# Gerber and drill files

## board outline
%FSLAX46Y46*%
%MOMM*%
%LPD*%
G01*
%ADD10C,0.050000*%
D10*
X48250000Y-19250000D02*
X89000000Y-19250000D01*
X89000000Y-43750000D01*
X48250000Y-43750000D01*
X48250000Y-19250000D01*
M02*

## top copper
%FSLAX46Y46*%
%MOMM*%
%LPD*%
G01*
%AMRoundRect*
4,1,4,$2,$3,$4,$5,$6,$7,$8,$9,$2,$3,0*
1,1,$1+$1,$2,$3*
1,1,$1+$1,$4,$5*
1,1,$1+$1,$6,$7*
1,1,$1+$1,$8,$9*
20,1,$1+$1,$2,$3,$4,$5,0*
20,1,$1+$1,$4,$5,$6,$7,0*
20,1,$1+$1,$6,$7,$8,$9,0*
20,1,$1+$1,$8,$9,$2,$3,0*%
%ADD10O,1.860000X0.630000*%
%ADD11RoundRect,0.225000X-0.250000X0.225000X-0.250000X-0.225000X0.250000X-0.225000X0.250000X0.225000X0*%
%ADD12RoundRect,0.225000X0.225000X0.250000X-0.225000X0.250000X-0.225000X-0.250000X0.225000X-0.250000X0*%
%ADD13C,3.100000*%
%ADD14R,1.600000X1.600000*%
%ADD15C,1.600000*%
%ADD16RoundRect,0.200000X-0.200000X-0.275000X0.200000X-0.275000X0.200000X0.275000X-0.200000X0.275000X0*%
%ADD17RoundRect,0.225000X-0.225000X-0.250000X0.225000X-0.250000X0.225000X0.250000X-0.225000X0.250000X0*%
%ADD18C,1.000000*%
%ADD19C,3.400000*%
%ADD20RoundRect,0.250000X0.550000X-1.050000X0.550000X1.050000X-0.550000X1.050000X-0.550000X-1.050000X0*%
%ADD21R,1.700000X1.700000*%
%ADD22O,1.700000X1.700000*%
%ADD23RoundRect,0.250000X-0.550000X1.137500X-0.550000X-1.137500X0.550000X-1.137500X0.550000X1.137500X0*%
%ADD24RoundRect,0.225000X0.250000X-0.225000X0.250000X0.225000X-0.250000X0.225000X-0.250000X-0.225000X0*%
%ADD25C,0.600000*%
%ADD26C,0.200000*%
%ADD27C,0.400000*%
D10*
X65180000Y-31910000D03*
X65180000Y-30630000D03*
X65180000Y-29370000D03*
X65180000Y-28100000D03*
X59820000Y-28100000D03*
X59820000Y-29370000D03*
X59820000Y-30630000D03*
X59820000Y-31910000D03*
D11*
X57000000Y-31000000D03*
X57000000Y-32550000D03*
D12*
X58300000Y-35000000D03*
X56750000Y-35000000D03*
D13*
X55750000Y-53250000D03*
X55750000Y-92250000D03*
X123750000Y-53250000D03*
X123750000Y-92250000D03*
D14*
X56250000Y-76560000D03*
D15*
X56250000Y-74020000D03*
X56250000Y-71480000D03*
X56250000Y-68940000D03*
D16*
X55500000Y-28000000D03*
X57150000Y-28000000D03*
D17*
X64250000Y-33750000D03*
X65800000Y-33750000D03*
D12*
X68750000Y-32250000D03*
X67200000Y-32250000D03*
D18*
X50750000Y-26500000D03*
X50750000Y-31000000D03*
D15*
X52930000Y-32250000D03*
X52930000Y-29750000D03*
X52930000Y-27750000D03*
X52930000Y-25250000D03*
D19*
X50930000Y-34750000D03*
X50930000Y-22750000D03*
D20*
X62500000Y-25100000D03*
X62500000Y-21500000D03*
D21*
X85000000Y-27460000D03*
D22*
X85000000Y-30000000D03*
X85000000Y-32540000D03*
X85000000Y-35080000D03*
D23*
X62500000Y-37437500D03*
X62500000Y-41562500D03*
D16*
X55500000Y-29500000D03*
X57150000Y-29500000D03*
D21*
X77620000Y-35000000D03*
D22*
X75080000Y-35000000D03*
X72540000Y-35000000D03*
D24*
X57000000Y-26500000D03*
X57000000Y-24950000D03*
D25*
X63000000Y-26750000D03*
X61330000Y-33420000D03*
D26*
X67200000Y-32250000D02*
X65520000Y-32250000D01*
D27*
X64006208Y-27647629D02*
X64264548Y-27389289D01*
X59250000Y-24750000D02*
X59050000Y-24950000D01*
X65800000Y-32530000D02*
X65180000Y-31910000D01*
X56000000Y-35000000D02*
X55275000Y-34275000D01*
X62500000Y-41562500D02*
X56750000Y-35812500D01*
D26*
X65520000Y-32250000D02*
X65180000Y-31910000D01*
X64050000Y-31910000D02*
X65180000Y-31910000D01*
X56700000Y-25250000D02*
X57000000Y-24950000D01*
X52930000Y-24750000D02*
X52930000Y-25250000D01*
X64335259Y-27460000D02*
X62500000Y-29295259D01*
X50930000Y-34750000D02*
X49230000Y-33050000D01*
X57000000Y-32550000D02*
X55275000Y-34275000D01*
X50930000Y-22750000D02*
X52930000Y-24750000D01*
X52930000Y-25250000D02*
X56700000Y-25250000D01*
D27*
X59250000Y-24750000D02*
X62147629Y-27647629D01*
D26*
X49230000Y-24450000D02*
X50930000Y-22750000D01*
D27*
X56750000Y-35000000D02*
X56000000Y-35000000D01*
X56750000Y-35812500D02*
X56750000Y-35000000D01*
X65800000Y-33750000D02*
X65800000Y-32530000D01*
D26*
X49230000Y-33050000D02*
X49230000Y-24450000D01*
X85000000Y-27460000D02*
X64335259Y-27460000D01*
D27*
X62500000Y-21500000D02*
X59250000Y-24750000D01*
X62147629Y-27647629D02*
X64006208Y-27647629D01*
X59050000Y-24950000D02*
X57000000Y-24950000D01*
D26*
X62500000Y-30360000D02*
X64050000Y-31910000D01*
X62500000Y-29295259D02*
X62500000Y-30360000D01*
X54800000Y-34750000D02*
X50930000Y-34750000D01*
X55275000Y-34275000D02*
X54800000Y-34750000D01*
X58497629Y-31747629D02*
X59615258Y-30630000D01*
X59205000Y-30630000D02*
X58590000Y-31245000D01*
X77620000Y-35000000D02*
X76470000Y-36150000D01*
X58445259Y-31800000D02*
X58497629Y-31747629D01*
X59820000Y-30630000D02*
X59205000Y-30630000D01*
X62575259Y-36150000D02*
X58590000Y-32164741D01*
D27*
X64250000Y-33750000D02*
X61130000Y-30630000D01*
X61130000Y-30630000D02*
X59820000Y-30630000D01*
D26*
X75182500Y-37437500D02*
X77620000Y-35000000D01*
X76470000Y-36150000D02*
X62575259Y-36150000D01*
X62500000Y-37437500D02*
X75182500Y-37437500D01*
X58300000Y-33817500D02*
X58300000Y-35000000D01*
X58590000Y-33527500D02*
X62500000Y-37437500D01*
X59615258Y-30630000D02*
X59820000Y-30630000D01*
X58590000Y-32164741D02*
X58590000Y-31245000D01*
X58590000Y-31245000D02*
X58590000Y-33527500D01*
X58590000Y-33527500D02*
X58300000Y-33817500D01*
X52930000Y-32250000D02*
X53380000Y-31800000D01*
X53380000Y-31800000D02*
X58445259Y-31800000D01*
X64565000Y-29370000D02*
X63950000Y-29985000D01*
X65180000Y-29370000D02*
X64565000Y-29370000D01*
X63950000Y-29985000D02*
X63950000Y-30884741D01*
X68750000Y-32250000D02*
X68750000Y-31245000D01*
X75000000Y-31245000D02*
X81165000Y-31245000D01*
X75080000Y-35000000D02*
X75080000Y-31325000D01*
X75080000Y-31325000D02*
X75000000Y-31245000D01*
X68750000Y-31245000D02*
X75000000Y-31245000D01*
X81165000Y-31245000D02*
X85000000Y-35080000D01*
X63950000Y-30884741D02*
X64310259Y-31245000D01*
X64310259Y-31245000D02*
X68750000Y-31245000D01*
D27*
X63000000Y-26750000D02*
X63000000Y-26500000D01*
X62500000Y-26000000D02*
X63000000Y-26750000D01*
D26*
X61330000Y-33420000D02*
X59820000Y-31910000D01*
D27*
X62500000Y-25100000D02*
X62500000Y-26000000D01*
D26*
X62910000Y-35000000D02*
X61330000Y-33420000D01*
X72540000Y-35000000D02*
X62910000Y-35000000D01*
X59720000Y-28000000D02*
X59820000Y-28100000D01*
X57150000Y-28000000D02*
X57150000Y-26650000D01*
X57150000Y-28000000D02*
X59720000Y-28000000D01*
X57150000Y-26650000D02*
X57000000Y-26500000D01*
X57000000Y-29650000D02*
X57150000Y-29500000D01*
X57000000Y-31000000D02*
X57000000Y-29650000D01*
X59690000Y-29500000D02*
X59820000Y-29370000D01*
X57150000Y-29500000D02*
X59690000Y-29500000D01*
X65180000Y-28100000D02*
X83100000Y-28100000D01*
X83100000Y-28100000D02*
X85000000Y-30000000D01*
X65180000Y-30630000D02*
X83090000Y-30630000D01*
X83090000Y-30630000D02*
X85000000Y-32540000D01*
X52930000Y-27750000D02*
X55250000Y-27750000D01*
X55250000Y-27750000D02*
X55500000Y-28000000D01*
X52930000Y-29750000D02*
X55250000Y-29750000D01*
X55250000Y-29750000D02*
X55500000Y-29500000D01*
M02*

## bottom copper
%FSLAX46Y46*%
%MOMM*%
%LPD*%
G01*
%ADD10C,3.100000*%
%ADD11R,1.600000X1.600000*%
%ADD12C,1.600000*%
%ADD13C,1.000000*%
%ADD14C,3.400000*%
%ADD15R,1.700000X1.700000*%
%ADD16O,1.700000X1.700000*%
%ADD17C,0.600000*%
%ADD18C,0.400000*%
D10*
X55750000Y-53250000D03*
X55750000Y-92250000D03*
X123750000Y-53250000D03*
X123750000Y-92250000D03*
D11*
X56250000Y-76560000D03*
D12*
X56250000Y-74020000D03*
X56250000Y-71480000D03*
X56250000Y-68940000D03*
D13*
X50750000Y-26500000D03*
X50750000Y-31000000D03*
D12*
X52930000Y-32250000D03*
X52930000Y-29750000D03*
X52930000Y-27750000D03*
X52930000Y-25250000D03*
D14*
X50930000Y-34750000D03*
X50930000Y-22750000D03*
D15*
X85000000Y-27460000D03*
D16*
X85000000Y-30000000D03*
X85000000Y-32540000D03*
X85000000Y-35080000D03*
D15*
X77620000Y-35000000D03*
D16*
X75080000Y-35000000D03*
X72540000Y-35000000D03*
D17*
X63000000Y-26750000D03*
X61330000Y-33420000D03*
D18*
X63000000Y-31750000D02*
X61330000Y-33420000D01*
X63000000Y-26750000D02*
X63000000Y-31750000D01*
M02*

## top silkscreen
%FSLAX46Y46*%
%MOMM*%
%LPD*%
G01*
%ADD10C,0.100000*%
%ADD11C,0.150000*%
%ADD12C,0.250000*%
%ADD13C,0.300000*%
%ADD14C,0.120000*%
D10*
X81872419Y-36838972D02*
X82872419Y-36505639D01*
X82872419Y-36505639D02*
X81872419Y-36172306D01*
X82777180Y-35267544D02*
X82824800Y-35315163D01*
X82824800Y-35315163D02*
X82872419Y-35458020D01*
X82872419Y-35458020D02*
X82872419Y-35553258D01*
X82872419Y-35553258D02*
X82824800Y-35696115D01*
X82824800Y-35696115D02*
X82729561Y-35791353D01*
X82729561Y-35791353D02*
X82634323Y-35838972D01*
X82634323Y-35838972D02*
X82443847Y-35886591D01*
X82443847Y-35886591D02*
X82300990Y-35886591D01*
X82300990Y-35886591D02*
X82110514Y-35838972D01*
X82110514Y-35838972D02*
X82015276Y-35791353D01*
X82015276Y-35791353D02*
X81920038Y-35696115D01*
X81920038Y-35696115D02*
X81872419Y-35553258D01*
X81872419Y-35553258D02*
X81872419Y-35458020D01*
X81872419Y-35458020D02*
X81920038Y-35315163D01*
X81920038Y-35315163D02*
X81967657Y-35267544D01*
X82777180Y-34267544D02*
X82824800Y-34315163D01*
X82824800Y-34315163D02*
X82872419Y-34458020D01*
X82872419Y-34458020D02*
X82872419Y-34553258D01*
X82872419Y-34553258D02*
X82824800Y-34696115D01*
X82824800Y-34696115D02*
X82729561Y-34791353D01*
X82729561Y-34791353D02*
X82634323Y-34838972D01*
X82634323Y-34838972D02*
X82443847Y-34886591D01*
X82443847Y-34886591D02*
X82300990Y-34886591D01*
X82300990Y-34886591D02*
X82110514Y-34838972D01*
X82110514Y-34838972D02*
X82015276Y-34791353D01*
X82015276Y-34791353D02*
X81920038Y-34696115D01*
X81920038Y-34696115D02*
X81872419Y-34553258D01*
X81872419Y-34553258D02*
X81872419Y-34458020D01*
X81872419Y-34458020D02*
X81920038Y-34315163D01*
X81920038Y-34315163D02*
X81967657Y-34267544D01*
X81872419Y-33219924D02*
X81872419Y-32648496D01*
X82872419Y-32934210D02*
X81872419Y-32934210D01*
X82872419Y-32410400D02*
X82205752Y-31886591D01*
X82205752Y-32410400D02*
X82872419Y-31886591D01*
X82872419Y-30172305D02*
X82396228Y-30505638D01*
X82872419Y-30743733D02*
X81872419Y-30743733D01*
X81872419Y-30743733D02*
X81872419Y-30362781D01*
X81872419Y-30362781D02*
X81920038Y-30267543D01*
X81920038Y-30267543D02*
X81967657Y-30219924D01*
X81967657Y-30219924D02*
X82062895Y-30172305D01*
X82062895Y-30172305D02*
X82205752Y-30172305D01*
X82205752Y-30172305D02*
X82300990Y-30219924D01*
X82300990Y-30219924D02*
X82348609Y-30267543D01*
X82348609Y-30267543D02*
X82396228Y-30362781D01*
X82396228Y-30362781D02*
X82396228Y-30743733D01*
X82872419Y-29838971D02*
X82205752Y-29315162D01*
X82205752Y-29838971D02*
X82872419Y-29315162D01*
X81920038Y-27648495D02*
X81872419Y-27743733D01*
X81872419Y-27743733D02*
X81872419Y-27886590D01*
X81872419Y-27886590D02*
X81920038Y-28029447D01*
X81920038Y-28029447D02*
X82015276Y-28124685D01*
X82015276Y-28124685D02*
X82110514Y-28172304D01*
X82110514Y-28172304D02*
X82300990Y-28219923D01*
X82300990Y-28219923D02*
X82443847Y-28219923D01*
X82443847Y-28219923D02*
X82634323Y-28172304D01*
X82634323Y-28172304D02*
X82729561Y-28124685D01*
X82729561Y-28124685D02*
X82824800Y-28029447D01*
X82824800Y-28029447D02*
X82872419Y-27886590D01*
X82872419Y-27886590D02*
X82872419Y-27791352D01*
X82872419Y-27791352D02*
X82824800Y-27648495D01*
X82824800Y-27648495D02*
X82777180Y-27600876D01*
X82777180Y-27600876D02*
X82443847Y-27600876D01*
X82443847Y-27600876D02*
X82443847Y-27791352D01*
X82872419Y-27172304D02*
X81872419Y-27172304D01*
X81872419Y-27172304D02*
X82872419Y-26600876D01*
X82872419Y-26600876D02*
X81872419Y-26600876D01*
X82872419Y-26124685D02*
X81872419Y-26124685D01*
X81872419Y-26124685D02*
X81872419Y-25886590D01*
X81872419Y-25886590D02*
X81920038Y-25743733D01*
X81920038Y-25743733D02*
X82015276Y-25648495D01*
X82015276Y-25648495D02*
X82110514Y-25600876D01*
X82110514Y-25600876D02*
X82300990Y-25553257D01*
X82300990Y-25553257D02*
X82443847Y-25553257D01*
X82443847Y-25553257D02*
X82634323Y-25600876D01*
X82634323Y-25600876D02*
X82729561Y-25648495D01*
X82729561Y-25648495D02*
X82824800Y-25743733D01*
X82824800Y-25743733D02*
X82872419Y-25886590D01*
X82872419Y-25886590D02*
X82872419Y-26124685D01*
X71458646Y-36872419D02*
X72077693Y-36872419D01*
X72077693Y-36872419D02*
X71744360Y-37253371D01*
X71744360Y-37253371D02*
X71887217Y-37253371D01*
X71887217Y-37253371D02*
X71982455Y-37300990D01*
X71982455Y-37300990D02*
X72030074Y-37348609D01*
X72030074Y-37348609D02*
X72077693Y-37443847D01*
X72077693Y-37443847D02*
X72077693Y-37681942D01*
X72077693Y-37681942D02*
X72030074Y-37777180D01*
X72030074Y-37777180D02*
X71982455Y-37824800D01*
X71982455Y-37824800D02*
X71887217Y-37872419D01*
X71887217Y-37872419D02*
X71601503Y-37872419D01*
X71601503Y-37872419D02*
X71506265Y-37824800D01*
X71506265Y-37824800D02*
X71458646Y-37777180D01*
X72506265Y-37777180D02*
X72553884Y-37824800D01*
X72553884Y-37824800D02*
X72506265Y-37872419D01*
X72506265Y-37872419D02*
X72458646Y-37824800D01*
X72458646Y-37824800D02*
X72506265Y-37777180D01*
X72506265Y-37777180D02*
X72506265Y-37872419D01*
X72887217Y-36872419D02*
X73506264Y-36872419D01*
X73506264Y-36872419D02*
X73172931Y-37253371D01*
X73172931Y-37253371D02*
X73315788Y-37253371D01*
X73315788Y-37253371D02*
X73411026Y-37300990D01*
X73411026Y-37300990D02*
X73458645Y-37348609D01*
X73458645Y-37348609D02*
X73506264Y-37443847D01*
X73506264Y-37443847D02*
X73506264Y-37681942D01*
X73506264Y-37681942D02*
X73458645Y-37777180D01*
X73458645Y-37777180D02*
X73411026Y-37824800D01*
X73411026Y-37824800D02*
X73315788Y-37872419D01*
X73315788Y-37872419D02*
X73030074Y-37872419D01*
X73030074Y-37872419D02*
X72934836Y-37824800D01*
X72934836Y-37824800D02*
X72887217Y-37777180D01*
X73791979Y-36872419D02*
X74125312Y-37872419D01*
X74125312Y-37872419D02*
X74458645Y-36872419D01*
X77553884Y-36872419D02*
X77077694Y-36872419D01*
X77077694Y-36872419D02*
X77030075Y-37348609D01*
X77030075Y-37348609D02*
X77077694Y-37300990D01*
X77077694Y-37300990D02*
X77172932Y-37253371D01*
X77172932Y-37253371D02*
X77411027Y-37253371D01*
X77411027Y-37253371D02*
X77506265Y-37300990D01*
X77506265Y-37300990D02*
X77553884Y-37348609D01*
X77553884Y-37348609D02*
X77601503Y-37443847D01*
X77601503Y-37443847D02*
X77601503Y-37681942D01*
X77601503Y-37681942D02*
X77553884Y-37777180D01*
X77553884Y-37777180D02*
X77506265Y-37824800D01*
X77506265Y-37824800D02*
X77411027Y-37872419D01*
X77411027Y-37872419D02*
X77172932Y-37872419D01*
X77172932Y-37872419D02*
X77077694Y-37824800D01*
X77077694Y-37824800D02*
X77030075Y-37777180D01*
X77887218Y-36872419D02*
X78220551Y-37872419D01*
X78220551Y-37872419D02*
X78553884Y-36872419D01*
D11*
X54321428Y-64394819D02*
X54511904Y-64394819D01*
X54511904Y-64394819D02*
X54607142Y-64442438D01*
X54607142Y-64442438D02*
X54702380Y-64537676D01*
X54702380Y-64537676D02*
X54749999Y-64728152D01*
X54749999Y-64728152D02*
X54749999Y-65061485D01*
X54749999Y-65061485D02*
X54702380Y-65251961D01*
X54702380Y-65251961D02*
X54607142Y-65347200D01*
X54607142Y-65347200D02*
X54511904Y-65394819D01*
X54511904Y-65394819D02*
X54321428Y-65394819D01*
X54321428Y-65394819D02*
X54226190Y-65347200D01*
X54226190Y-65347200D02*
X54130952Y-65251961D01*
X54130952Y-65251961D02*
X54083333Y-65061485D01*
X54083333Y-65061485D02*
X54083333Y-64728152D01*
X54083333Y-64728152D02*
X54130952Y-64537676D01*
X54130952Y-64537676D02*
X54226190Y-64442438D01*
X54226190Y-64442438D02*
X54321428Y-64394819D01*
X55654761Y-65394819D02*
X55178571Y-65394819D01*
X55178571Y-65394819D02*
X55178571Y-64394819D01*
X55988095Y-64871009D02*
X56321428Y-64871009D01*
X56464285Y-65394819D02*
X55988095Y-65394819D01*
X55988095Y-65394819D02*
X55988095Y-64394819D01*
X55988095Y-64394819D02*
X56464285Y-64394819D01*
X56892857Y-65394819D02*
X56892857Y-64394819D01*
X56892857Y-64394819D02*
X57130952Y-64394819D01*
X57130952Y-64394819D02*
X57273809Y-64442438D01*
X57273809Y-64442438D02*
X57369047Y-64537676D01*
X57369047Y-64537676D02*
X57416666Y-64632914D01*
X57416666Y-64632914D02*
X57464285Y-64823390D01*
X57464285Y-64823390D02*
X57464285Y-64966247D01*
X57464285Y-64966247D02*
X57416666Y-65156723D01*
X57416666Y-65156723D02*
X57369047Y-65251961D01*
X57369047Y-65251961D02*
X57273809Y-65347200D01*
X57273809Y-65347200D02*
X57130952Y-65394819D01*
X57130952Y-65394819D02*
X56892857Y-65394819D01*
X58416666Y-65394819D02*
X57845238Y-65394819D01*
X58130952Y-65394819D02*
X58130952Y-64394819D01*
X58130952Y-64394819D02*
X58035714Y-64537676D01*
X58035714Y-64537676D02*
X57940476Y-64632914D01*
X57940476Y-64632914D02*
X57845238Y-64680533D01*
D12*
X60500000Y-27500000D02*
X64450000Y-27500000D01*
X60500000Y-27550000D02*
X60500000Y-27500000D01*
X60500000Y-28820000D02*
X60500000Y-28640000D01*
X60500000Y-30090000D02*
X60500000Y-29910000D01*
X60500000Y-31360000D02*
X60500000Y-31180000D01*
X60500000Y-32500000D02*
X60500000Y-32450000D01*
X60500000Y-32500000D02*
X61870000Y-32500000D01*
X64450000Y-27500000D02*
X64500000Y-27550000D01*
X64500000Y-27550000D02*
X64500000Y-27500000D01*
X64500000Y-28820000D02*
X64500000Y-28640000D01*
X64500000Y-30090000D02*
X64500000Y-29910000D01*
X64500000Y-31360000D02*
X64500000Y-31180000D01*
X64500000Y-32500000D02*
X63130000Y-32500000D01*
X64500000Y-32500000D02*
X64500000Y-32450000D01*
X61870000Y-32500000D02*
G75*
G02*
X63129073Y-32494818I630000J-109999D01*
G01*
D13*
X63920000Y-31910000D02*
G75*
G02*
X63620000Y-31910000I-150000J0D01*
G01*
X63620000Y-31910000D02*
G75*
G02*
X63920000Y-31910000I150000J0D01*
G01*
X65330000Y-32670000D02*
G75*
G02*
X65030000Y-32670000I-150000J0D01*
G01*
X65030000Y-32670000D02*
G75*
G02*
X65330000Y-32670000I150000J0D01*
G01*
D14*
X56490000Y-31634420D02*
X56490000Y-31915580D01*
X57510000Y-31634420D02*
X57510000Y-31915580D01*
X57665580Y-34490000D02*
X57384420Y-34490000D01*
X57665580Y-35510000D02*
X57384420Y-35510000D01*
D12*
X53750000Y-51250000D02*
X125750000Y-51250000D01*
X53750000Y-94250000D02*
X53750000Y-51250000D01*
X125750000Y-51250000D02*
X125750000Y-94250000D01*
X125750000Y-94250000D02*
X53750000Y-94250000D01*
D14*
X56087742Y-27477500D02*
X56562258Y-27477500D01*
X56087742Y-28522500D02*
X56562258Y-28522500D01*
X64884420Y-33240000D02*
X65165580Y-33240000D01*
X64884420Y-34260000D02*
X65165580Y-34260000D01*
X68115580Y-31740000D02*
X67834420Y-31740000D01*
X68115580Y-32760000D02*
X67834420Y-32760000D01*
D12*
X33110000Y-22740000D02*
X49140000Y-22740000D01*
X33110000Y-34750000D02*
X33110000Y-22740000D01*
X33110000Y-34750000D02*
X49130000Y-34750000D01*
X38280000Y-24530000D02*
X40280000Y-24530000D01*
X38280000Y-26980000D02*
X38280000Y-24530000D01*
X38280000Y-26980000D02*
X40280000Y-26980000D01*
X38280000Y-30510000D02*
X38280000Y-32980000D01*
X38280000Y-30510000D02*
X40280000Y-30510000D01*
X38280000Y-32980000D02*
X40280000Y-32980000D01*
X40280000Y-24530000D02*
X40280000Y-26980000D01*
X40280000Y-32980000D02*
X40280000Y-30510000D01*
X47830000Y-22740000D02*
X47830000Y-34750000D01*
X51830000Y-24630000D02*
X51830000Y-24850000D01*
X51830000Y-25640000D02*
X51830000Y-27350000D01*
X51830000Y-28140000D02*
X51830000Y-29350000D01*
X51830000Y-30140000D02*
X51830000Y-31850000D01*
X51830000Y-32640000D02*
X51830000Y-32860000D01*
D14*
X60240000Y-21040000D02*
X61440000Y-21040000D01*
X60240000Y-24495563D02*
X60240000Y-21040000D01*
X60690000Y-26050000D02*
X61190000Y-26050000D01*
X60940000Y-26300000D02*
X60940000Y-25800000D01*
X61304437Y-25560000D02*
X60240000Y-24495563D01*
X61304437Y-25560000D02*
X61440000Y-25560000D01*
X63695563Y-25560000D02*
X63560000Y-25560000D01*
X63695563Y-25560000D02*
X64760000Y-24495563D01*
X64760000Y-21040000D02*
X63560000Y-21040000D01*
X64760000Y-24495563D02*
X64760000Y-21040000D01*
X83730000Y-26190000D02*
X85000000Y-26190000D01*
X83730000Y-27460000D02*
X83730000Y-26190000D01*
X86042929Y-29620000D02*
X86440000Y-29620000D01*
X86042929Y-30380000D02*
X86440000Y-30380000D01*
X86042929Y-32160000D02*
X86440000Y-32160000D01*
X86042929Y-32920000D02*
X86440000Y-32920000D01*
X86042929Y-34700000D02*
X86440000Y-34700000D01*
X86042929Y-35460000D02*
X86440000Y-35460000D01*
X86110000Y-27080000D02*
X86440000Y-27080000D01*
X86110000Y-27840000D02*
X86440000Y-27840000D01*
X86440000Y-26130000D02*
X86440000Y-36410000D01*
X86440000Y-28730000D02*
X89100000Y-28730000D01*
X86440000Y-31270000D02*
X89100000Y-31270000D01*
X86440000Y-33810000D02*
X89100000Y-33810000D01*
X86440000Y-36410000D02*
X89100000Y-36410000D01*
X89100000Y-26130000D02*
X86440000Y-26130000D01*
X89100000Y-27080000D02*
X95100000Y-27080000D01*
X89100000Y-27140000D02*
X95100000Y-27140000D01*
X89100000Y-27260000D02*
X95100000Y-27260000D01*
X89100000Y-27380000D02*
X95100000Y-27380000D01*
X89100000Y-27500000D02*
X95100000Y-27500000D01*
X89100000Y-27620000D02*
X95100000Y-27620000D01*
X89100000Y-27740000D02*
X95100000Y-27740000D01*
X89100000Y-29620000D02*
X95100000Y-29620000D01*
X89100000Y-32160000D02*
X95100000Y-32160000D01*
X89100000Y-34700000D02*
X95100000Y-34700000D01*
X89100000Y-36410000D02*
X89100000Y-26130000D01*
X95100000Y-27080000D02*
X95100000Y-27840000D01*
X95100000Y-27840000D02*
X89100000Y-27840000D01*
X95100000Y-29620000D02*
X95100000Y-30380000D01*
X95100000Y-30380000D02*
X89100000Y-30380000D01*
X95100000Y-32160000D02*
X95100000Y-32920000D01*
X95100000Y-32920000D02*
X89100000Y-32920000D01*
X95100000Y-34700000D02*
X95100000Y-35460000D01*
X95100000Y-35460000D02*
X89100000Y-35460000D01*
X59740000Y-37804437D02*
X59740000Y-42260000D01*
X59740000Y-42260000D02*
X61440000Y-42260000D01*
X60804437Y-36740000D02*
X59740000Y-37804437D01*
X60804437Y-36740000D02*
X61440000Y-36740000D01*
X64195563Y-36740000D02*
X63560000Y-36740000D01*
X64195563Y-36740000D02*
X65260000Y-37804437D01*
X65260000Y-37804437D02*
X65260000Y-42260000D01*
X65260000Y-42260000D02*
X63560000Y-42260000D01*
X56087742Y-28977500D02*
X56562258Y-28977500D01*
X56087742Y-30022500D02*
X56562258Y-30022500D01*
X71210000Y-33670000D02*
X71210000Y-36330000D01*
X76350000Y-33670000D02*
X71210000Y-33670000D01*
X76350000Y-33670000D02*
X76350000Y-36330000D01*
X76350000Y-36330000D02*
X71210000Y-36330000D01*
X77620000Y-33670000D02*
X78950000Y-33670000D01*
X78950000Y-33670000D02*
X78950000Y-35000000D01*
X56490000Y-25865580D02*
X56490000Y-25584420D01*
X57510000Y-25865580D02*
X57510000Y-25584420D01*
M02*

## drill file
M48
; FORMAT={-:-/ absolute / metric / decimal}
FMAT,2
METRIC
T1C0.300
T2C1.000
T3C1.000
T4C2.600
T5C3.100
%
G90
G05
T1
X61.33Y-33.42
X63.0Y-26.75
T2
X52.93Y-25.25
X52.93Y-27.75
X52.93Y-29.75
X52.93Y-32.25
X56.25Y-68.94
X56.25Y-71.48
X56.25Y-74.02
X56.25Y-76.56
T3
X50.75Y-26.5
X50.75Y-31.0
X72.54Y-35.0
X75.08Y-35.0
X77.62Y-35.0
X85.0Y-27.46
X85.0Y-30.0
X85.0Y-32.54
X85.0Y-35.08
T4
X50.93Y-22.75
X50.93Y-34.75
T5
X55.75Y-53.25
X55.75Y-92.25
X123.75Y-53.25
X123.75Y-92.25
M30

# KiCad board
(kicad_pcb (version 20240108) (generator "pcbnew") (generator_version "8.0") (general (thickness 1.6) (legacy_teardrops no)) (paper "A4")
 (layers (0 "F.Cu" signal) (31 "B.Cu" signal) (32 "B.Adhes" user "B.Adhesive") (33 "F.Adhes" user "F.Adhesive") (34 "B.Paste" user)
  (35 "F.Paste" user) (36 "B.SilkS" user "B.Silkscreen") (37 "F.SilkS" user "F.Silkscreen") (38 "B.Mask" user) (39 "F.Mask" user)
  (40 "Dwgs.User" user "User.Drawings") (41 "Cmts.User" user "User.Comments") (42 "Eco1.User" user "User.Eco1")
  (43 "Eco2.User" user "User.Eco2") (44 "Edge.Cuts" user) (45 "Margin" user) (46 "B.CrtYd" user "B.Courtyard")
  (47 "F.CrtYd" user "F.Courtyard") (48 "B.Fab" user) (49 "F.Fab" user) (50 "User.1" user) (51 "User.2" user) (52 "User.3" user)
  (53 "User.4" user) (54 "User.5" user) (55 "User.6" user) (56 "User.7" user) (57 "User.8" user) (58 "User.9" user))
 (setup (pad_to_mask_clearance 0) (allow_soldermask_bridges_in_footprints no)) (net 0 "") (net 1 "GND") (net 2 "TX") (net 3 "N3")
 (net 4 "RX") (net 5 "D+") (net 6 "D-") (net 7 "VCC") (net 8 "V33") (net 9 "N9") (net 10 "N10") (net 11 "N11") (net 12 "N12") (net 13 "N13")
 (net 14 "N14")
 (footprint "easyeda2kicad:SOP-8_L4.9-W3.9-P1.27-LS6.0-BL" (layer "F.Cu") (at 62.5 30 90)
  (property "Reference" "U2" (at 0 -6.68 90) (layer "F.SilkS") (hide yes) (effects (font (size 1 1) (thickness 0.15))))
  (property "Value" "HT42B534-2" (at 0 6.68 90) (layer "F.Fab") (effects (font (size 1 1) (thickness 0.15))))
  (fp_line (start 2.5 -2) (end 2.5 1.95) (stroke (width 0.25) (type solid)) (layer "F.SilkS"))
  (fp_line (start 2.45 -2) (end 2.5 -2) (stroke (width 0.25) (type solid)) (layer "F.SilkS"))
  (fp_line (start 1.18 -2) (end 1.36 -2) (stroke (width 0.25) (type solid)) (layer "F.SilkS"))
  (fp_line (start -0.09 -2) (end 0.09 -2) (stroke (width 0.25) (type solid)) (layer "F.SilkS"))
  (fp_line (start -1.36 -2) (end -1.18 -2) (stroke (width 0.25) (type solid)) (layer "F.SilkS"))
  (fp_line (start -2.5 -2) (end -2.45 -2) (stroke (width 0.25) (type solid)) (layer "F.SilkS"))
  (fp_line (start -2.5 -2) (end -2.5 -0.63) (stroke (width 0.25) (type solid)) (layer "F.SilkS"))
  (fp_line (start 2.5 1.95) (end 2.45 2) (stroke (width 0.25) (type solid)) (layer "F.SilkS"))
  (fp_line (start 2.45 2) (end 2.5 2) (stroke (width 0.25) (type solid)) (layer "F.SilkS"))
  (fp_line (start 1.18 2) (end 1.36 2) (stroke (width 0.25) (type solid)) (layer "F.SilkS"))
  (fp_line (start -0.09 2) (end 0.09 2) (stroke (width 0.25) (type solid)) (layer "F.SilkS"))
  (fp_line (start -1.36 2) (end -1.18 2) (stroke (width 0.25) (type solid)) (layer "F.SilkS"))
  (fp_line (start -2.5 2) (end -2.5 0.63) (stroke (width 0.25) (type solid)) (layer "F.SilkS"))
  (fp_line (start -2.5 2) (end -2.45 2) (stroke (width 0.25) (type solid)) (layer "F.SilkS"))
  (fp_arc (start -2.5 -0.63) (mid -1.970474 -0.002632) (end -2.494818 0.629073) (stroke (width 0.25) (type solid)) (layer "F.SilkS"))
  (fp_circle (center -1.91 1.27) (end -1.76 1.27) (stroke (width 0.3) (type solid)) (fill none) (layer "F.SilkS"))
  (fp_circle (center -2.67 2.68) (end -2.52 2.68) (stroke (width 0.3) (type solid)) (fill none) (layer "F.SilkS"))
  (pad "1" smd oval (at -1.91 2.68 90) (size 0.63 1.86) (layers "F.Cu" "F.Paste" "F.Mask") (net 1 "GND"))
  (pad "2" smd oval (at -0.63 2.68 90) (size 0.63 1.86) (layers "F.Cu" "F.Paste" "F.Mask") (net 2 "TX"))
  (pad "3" smd oval (at 0.63 2.68 90) (size 0.63 1.86) (layers "F.Cu" "F.Paste" "F.Mask") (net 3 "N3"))
  (pad "4" smd oval (at 1.9 2.68 90) (size 0.63 1.86) (layers "F.Cu" "F.Paste" "F.Mask") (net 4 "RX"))
  (pad "5" smd oval (at 1.9 -2.68 90) (size 0.63 1.86) (layers "F.Cu" "F.Paste" "F.Mask") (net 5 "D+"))
  (pad "6" smd oval (at 0.63 -2.68 90) (size 0.63 1.86) (layers "F.Cu" "F.Paste" "F.Mask") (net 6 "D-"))
  (pad "7" smd oval (at -0.63 -2.68 90) (size 0.63 1.86) (layers "F.Cu" "F.Paste" "F.Mask") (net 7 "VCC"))
  (pad "8" smd oval (at -1.91 -2.68 90) (size 0.63 1.86) (layers "F.Cu" "F.Paste" "F.Mask") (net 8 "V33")))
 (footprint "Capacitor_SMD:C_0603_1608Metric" (layer "F.Cu") (at 57 31.775 -90)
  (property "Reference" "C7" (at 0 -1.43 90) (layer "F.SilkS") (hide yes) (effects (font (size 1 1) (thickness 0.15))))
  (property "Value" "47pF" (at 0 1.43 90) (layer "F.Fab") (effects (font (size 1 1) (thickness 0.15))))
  (fp_line (start -0.14058 0.51) (end 0.14058 0.51) (stroke (width 0.12) (type solid)) (layer "F.SilkS"))
  (fp_line (start -0.14058 -0.51) (end 0.14058 -0.51) (stroke (width 0.12) (type solid)) (layer "F.SilkS"))
  (pad "1" smd roundrect (at -0.775 0 270) (size 0.9 0.95) (layers "F.Cu" "F.Paste" "F.Mask") (roundrect_rratio 0.25) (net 6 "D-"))
  (pad "2" smd roundrect (at 0.775 0 270) (size 0.9 0.95) (layers "F.Cu" "F.Paste" "F.Mask") (roundrect_rratio 0.25) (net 1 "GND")))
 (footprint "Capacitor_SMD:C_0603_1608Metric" (layer "F.Cu") (at 57.525 35 180)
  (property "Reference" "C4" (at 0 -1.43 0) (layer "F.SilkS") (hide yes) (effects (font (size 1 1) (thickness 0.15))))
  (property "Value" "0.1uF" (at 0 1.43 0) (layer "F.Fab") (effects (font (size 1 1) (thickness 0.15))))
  (fp_line (start -0.14058 0.51) (end 0.14058 0.51) (stroke (width 0.12) (type solid)) (layer "F.SilkS"))
  (fp_line (start -0.14058 -0.51) (end 0.14058 -0.51) (stroke (width 0.12) (type solid)) (layer "F.SilkS"))
  (pad "1" smd roundrect (at -0.775 0 180) (size 0.9 0.95) (layers "F.Cu" "F.Paste" "F.Mask") (roundrect_rratio 0.25) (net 7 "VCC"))
  (pad "2" smd roundrect (at 0.775 0 180) (size 0.9 0.95) (layers "F.Cu" "F.Paste" "F.Mask") (roundrect_rratio 0.25) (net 1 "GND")))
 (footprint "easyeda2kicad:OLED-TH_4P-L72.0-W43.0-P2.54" (layer "F.Cu") (at 56.25 72.75)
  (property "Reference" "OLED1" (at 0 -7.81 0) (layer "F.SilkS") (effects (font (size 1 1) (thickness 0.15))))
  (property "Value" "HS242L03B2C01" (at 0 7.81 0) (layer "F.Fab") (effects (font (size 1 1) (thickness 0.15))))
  (fp_line (start -2.5 -21.5) (end 69.5 -21.5) (stroke (width 0.25) (type solid)) (layer "F.SilkS"))
  (fp_line (start -2.5 21.5) (end -2.5 -21.5) (stroke (width 0.25) (type solid)) (layer "F.SilkS"))
  (fp_line (start 69.5 -21.5) (end 69.5 21.5) (stroke (width 0.25) (type solid)) (layer "F.SilkS"))
  (fp_line (start 69.5 21.5) (end -2.5 21.5) (stroke (width 0.25) (type solid)) (layer "F.SilkS"))
  (pad "" thru_hole circle (at -0.5 -19.5) (size 3.1 3.1) (drill 3.1) (layers "*.Cu" "*.Mask") (remove_unused_layers no))
  (pad "" thru_hole circle (at -0.5 19.5) (size 3.1 3.1) (drill 3.1) (layers "*.Cu" "*.Mask") (remove_unused_layers no))
  (pad "" thru_hole circle (at 67.5 -19.5) (size 3.1 3.1) (drill 3.1) (layers "*.Cu" "*.Mask") (remove_unused_layers no))
  (pad "" thru_hole circle (at 67.5 19.5) (size 3.1 3.1) (drill 3.1) (layers "*.Cu" "*.Mask") (remove_unused_layers no))
  (pad "1" thru_hole rect (at 0 3.81) (size 1.6 1.6) (drill 0.999998) (layers "*.Cu" "*.Mask") (remove_unused_layers no) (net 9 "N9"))
  (pad "2" thru_hole circle (at 0 1.27) (size 1.6 1.6) (drill 0.999998) (layers "*.Cu" "*.Mask") (remove_unused_layers no) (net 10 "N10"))
  (pad "3" thru_hole circle (at 0 -1.27) (size 1.6 1.6) (drill 0.999998) (layers "*.Cu" "*.Mask") (remove_unused_layers no) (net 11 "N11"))
  (pad "4" thru_hole circle (at 0 -3.81) (size 1.6 1.6) (drill 0.999998) (layers "*.Cu" "*.Mask") (remove_unused_layers no) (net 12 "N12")))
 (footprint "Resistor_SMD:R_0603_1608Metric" (layer "F.Cu") (at 56.325 28)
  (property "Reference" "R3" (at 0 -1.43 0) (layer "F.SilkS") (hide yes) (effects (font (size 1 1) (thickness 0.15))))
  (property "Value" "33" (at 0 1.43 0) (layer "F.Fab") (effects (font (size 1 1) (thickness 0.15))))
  (fp_line (start -0.237258 -0.5225) (end 0.237258 -0.5225) (stroke (width 0.12) (type solid)) (layer "F.SilkS"))
  (fp_line (start -0.237258 0.5225) (end 0.237258 0.5225) (stroke (width 0.12) (type solid)) (layer "F.SilkS"))
  (pad "1" smd roundrect (at -0.825 0) (size 0.8 0.95) (layers "F.Cu" "F.Paste" "F.Mask") (roundrect_rratio 0.25) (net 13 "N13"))
  (pad "2" smd roundrect (at 0.825 0) (size 0.8 0.95) (layers "F.Cu" "F.Paste" "F.Mask") (roundrect_rratio 0.25) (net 5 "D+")))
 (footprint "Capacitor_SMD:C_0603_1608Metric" (layer "F.Cu") (at 65.025 33.75)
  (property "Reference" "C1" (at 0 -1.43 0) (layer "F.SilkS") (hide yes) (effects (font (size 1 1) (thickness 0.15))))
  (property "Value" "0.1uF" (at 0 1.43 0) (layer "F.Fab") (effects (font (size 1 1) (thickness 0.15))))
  (fp_line (start -0.14058 -0.51) (end 0.14058 -0.51) (stroke (width 0.12) (type solid)) (layer "F.SilkS"))
  (fp_line (start -0.14058 0.51) (end 0.14058 0.51) (stroke (width 0.12) (type solid)) (layer "F.SilkS"))
  (pad "1" smd roundrect (at -0.775 0) (size 0.9 0.95) (layers "F.Cu" "F.Paste" "F.Mask") (roundrect_rratio 0.25) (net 7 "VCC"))
  (pad "2" smd roundrect (at 0.775 0) (size 0.9 0.95) (layers "F.Cu" "F.Paste" "F.Mask") (roundrect_rratio 0.25) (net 1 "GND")))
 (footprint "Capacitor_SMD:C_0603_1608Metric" (layer "F.Cu") (at 67.975 32.25 180)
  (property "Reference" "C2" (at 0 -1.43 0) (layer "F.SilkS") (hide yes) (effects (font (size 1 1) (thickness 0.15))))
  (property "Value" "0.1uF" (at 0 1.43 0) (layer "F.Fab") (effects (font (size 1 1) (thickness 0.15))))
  (fp_line (start -0.14058 0.51) (end 0.14058 0.51) (stroke (width 0.12) (type solid)) (layer "F.SilkS"))
  (fp_line (start -0.14058 -0.51) (end 0.14058 -0.51) (stroke (width 0.12) (type solid)) (layer "F.SilkS"))
  (pad "1" smd roundrect (at -0.775 0 180) (size 0.9 0.95) (layers "F.Cu" "F.Paste" "F.Mask") (roundrect_rratio 0.25) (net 3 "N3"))
  (pad "2" smd roundrect (at 0.775 0 180) (size 0.9 0.95) (layers "F.Cu" "F.Paste" "F.Mask") (roundrect_rratio 0.25) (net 1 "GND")))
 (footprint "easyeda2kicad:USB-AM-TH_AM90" (layer "F.Cu") (at 51.93 28.75 -90)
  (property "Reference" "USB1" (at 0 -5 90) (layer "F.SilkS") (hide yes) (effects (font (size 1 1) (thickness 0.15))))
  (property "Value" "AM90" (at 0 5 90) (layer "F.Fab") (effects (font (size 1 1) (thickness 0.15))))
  (fp_line (start -6.01 18.82) (end -6.01 2.79) (stroke (width 0.25) (type solid)) (layer "F.SilkS"))
  (fp_line (start 6 18.82) (end -6.01 18.82) (stroke (width 0.25) (type solid)) (layer "F.SilkS"))
  (fp_line (start 6 18.82) (end 6 2.8) (stroke (width 0.25) (type solid)) (layer "F.SilkS"))
  (fp_line (start -4.22 13.65) (end -4.22 11.65) (stroke (width 0.25) (type solid)) (layer "F.SilkS"))
  (fp_line (start -1.77 13.65) (end -4.22 13.65) (stroke (width 0.25) (type solid)) (layer "F.SilkS"))
  (fp_line (start -1.77 13.65) (end -1.77 11.65) (stroke (width 0.25) (type solid)) (layer "F.SilkS"))
  (fp_line (start 1.76 13.65) (end 4.23 13.65) (stroke (width 0.25) (type solid)) (layer "F.SilkS"))
  (fp_line (start 1.76 13.65) (end 1.76 11.65) (stroke (width 0.25) (type solid)) (layer "F.SilkS"))
  (fp_line (start 4.23 13.65) (end 4.23 11.65) (stroke (width 0.25) (type solid)) (layer "F.SilkS"))
  (fp_line (start -4.22 11.65) (end -1.77 11.65) (stroke (width 0.25) (type solid)) (layer "F.SilkS"))
  (fp_line (start 4.23 11.65) (end 1.76 11.65) (stroke (width 0.25) (type solid)) (layer "F.SilkS"))
  (fp_line (start -6.01 4.1) (end 6 4.1) (stroke (width 0.25) (type solid)) (layer "F.SilkS"))
  (fp_line (start -4.12 0.1) (end -3.9 0.1) (stroke (width 0.25) (type solid)) (layer "F.SilkS"))
  (fp_line (start -3.11 0.1) (end -1.4 0.1) (stroke (width 0.25) (type solid)) (layer "F.SilkS"))
  (fp_line (start -0.61 0.1) (end 0.6 0.1) (stroke (width 0.25) (type solid)) (layer "F.SilkS"))
  (fp_line (start 1.39 0.1) (end 3.1 0.1) (stroke (width 0.25) (type solid)) (layer "F.SilkS"))
  (fp_line (start 3.89 0.1) (end 4.11 0.1) (stroke (width 0.25) (type solid)) (layer "F.SilkS"))
  (pad "" thru_hole circle (at -2.25 1.18 270) (size 1 1) (drill 1) (layers "*.Cu" "*.Mask") (remove_unused_layers no))
  (pad "" thru_hole circle (at 2.25 1.18 270) (size 1 1) (drill 1) (layers "*.Cu" "*.Mask") (remove_unused_layers no))
  (pad "1" thru_hole circle (at 3.5 -1 180) (size 1.6 1.6) (drill 0.999998) (layers "*.Cu" "*.Mask") (remove_unused_layers no) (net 7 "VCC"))
  (pad "2" thru_hole circle (at 1 -1 180) (size 1.6 1.6) (drill 0.999998) (layers "*.Cu" "*.Mask") (remove_unused_layers no) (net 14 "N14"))
  (pad "3" thru_hole circle (at -1 -1 180) (size 1.6 1.6) (drill 0.999998) (layers "*.Cu" "*.Mask") (remove_unused_layers no) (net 13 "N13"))
  (pad "4" thru_hole circle (at -3.5 -1 180) (size 1.6 1.6) (drill 0.999998) (layers "*.Cu" "*.Mask") (remove_unused_layers no)
   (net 1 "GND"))
  (pad "MH1" thru_hole circle (at 6 1 180) (size 3.4 3.4) (drill 2.599995) (layers "*.Cu" "*.Mask") (remove_unused_layers no) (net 1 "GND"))
  (pad "MH2" thru_hole circle (at -6 1 180) (size 3.4 3.4) (drill 2.599995) (layers "*.Cu" "*.Mask") (remove_unused_layers no) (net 1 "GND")))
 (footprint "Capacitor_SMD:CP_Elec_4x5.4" (layer "F.Cu") (at 62.5 23.3 90)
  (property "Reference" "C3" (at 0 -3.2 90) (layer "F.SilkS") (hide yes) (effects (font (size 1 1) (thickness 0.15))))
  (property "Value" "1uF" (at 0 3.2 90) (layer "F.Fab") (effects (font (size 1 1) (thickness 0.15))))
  (fp_line (start 2.26 -2.26) (end 2.26 -1.06) (stroke (width 0.12) (type solid)) (layer "F.SilkS"))
  (fp_line (start -1.195563 -2.26) (end 2.26 -2.26) (stroke (width 0.12) (type solid)) (layer "F.SilkS"))
  (fp_line (start -2.75 -1.81) (end -2.75 -1.31) (stroke (width 0.12) (type solid)) (layer "F.SilkS"))
  (fp_line (start -3 -1.56) (end -2.5 -1.56) (stroke (width 0.12) (type solid)) (layer "F.SilkS"))
  (fp_line (start -2.26 -1.195563) (end -1.195563 -2.26) (stroke (width 0.12) (type solid)) (layer "F.SilkS"))
  (fp_line (start -2.26 -1.195563) (end -2.26 -1.06) (stroke (width 0.12) (type solid)) (layer "F.SilkS"))
  (fp_line (start -2.26 1.195563) (end -2.26 1.06) (stroke (width 0.12) (type solid)) (layer "F.SilkS"))
  (fp_line (start -2.26 1.195563) (end -1.195563 2.26) (stroke (width 0.12) (type solid)) (layer "F.SilkS"))
  (fp_line (start 2.26 2.26) (end 2.26 1.06) (stroke (width 0.12) (type solid)) (layer "F.SilkS"))
  (fp_line (start -1.195563 2.26) (end 2.26 2.26) (stroke (width 0.12) (type solid)) (layer "F.SilkS"))
  (pad "1" smd roundrect (at -1.8 0 90) (size 2.6 1.6) (layers "F.Cu" "F.Paste" "F.Mask") (roundrect_rratio 0.15625) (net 8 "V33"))
  (pad "2" smd roundrect (at 1.8 0 90) (size 2.6 1.6) (layers "F.Cu" "F.Paste" "F.Mask") (roundrect_rratio 0.15625) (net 1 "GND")))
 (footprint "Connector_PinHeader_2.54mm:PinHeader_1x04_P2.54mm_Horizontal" (layer "F.Cu") (at 85 27.46)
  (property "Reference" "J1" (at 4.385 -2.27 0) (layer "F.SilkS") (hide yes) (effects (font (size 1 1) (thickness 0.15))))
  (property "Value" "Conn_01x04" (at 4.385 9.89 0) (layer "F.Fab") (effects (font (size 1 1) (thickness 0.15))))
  (fp_line (start -1.27 -1.27) (end 0 -1.27) (stroke (width 0.12) (type solid)) (layer "F.SilkS"))
  (fp_line (start -1.27 0) (end -1.27 -1.27) (stroke (width 0.12) (type solid)) (layer "F.SilkS"))
  (fp_line (start 1.042929 2.16) (end 1.44 2.16) (stroke (width 0.12) (type solid)) (layer "F.SilkS"))
  (fp_line (start 1.042929 2.92) (end 1.44 2.92) (stroke (width 0.12) (type solid)) (layer "F.SilkS"))
  (fp_line (start 1.042929 4.7) (end 1.44 4.7) (stroke (width 0.12) (type solid)) (layer "F.SilkS"))
  (fp_line (start 1.042929 5.46) (end 1.44 5.46) (stroke (width 0.12) (type solid)) (layer "F.SilkS"))
  (fp_line (start 1.042929 7.24) (end 1.44 7.24) (stroke (width 0.12) (type solid)) (layer "F.SilkS"))
  (fp_line (start 1.042929 8) (end 1.44 8) (stroke (width 0.12) (type solid)) (layer "F.SilkS"))
  (fp_line (start 1.11 -0.38) (end 1.44 -0.38) (stroke (width 0.12) (type solid)) (layer "F.SilkS"))
  (fp_line (start 1.11 0.38) (end 1.44 0.38) (stroke (width 0.12) (type solid)) (layer "F.SilkS"))
  (fp_line (start 1.44 -1.33) (end 1.44 8.95) (stroke (width 0.12) (type solid)) (layer "F.SilkS"))
  (fp_line (start 1.44 1.27) (end 4.1 1.27) (stroke (width 0.12) (type solid)) (layer "F.SilkS"))
  (fp_line (start 1.44 3.81) (end 4.1 3.81) (stroke (width 0.12) (type solid)) (layer "F.SilkS"))
  (fp_line (start 1.44 6.35) (end 4.1 6.35) (stroke (width 0.12) (type solid)) (layer "F.SilkS"))
  (fp_line (start 1.44 8.95) (end 4.1 8.95) (stroke (width 0.12) (type solid)) (layer "F.SilkS"))
  (fp_line (start 4.1 -1.33) (end 1.44 -1.33) (stroke (width 0.12) (type solid)) (layer "F.SilkS"))
  (fp_line (start 4.1 -0.38) (end 10.1 -0.38) (stroke (width 0.12) (type solid)) (layer "F.SilkS"))
  (fp_line (start 4.1 -0.32) (end 10.1 -0.32) (stroke (width 0.12) (type solid)) (layer "F.SilkS"))
  (fp_line (start 4.1 -0.2) (end 10.1 -0.2) (stroke (width 0.12) (type solid)) (layer "F.SilkS"))
  (fp_line (start 4.1 -0.08) (end 10.1 -0.08) (stroke (width 0.12) (type solid)) (layer "F.SilkS"))
  (fp_line (start 4.1 0.04) (end 10.1 0.04) (stroke (width 0.12) (type solid)) (layer "F.SilkS"))
  (fp_line (start 4.1 0.16) (end 10.1 0.16) (stroke (width 0.12) (type solid)) (layer "F.SilkS"))
  (fp_line (start 4.1 0.28) (end 10.1 0.28) (stroke (width 0.12) (type solid)) (layer "F.SilkS"))
  (fp_line (start 4.1 2.16) (end 10.1 2.16) (stroke (width 0.12) (type solid)) (layer "F.SilkS"))
  (fp_line (start 4.1 4.7) (end 10.1 4.7) (stroke (width 0.12) (type solid)) (layer "F.SilkS"))
  (fp_line (start 4.1 7.24) (end 10.1 7.24) (stroke (width 0.12) (type solid)) (layer "F.SilkS"))
  (fp_line (start 4.1 8.95) (end 4.1 -1.33) (stroke (width 0.12) (type solid)) (layer "F.SilkS"))
  (fp_line (start 10.1 -0.38) (end 10.1 0.38) (stroke (width 0.12) (type solid)) (layer "F.SilkS"))
  (fp_line (start 10.1 0.38) (end 4.1 0.38) (stroke (width 0.12) (type solid)) (layer "F.SilkS"))
  (fp_line (start 10.1 2.16) (end 10.1 2.92) (stroke (width 0.12) (type solid)) (layer "F.SilkS"))
  (fp_line (start 10.1 2.92) (end 4.1 2.92) (stroke (width 0.12) (type solid)) (layer "F.SilkS"))
  (fp_line (start 10.1 4.7) (end 10.1 5.46) (stroke (width 0.12) (type solid)) (layer "F.SilkS"))
  (fp_line (start 10.1 5.46) (end 4.1 5.46) (stroke (width 0.12) (type solid)) (layer "F.SilkS"))
  (fp_line (start 10.1 7.24) (end 10.1 8) (stroke (width 0.12) (type solid)) (layer "F.SilkS"))
  (fp_line (start 10.1 8) (end 4.1 8) (stroke (width 0.12) (type solid)) (layer "F.SilkS"))
  (pad "1" thru_hole rect (at 0 0) (size 1.7 1.7) (drill 1) (layers "*.Cu" "*.Mask") (remove_unused_layers no) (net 1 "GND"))
  (pad "2" thru_hole oval (at 0 2.54) (size 1.7 1.7) (drill 1) (layers "*.Cu" "*.Mask") (remove_unused_layers no) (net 4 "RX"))
  (pad "3" thru_hole oval (at 0 5.08) (size 1.7 1.7) (drill 1) (layers "*.Cu" "*.Mask") (remove_unused_layers no) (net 2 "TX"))
  (pad "4" thru_hole oval (at 0 7.62) (size 1.7 1.7) (drill 1) (layers "*.Cu" "*.Mask") (remove_unused_layers no) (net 3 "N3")))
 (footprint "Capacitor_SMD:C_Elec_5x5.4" (layer "F.Cu") (at 62.5 39.5 -90)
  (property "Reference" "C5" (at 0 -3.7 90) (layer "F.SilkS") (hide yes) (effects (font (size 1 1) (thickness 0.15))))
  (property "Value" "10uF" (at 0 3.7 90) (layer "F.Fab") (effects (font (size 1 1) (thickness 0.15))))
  (fp_line (start -1.695563 2.76) (end 2.76 2.76) (stroke (width 0.12) (type solid)) (layer "F.SilkS"))
  (fp_line (start 2.76 2.76) (end 2.76 1.06) (stroke (width 0.12) (type solid)) (layer "F.SilkS"))
  (fp_line (start -2.76 1.695563) (end -1.695563 2.76) (stroke (width 0.12) (type solid)) (layer "F.SilkS"))
  (fp_line (start -2.76 1.695563) (end -2.76 1.06) (stroke (width 0.12) (type solid)) (layer "F.SilkS"))
  (fp_line (start -2.76 -1.695563) (end -2.76 -1.06) (stroke (width 0.12) (type solid)) (layer "F.SilkS"))
  (fp_line (start -2.76 -1.695563) (end -1.695563 -2.76) (stroke (width 0.12) (type solid)) (layer "F.SilkS"))
  (fp_line (start -1.695563 -2.76) (end 2.76 -2.76) (stroke (width 0.12) (type solid)) (layer "F.SilkS"))
  (fp_line (start 2.76 -2.76) (end 2.76 -1.06) (stroke (width 0.12) (type solid)) (layer "F.SilkS"))
  (pad "1" smd roundrect (at -2.0625 0 270) (size 2.775 1.6) (layers "F.Cu" "F.Paste" "F.Mask") (roundrect_rratio 0.15625) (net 7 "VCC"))
  (pad "2" smd roundrect (at 2.0625 0 270) (size 2.775 1.6) (layers "F.Cu" "F.Paste" "F.Mask") (roundrect_rratio 0.15625) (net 1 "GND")))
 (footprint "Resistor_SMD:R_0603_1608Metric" (layer "F.Cu") (at 56.325 29.5)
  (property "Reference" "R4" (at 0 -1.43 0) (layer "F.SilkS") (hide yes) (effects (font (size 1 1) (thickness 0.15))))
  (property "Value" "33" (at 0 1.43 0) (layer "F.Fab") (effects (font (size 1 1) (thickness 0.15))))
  (fp_line (start -0.237258 -0.5225) (end 0.237258 -0.5225) (stroke (width 0.12) (type solid)) (layer "F.SilkS"))
  (fp_line (start -0.237258 0.5225) (end 0.237258 0.5225) (stroke (width 0.12) (type solid)) (layer "F.SilkS"))
  (pad "1" smd roundrect (at -0.825 0) (size 0.8 0.95) (layers "F.Cu" "F.Paste" "F.Mask") (roundrect_rratio 0.25) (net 14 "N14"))
  (pad "2" smd roundrect (at 0.825 0) (size 0.8 0.95) (layers "F.Cu" "F.Paste" "F.Mask") (roundrect_rratio 0.25) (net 6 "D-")))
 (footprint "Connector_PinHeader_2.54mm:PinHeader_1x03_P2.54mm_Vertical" (layer "F.Cu") (at 77.62 35 -90)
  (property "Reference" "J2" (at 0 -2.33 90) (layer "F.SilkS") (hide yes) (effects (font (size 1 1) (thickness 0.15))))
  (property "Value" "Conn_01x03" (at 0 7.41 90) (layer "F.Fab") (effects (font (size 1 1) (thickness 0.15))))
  (fp_line (start -1.33 6.41) (end 1.33 6.41) (stroke (width 0.12) (type solid)) (layer "F.SilkS"))
  (fp_line (start -1.33 1.27) (end -1.33 6.41) (stroke (width 0.12) (type solid)) (layer "F.SilkS"))
  (fp_line (start -1.33 1.27) (end 1.33 1.27) (stroke (width 0.12) (type solid)) (layer "F.SilkS"))
  (fp_line (start 1.33 1.27) (end 1.33 6.41) (stroke (width 0.12) (type solid)) (layer "F.SilkS"))
  (fp_line (start -1.33 0) (end -1.33 -1.33) (stroke (width 0.12) (type solid)) (layer "F.SilkS"))
  (fp_line (start -1.33 -1.33) (end 0 -1.33) (stroke (width 0.12) (type solid)) (layer "F.SilkS"))
  (pad "1" thru_hole rect (at 0 0 270) (size 1.7 1.7) (drill 1) (layers "*.Cu" "*.Mask") (remove_unused_layers no) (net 7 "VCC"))
  (pad "2" thru_hole oval (at 0 2.54 270) (size 1.7 1.7) (drill 1) (layers "*.Cu" "*.Mask") (remove_unused_layers no) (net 3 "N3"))
  (pad "3" thru_hole oval (at 0 5.08 270) (size 1.7 1.7) (drill 1) (layers "*.Cu" "*.Mask") (remove_unused_layers no) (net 8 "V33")))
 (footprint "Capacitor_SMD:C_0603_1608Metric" (layer "F.Cu") (at 57 25.725 90)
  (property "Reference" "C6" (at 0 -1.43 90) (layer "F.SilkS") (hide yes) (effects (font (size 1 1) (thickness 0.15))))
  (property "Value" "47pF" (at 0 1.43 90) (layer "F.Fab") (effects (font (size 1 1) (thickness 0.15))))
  (fp_line (start -0.14058 -0.51) (end 0.14058 -0.51) (stroke (width 0.12) (type solid)) (layer "F.SilkS"))
  (fp_line (start -0.14058 0.51) (end 0.14058 0.51) (stroke (width 0.12) (type solid)) (layer "F.SilkS"))
  (pad "1" smd roundrect (at -0.775 0 90) (size 0.9 0.95) (layers "F.Cu" "F.Paste" "F.Mask") (roundrect_rratio 0.25) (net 5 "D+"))
  (pad "2" smd roundrect (at 0.775 0 90) (size 0.9 0.95) (layers "F.Cu" "F.Paste" "F.Mask") (roundrect_rratio 0.25) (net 1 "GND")))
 (gr_rect (start 48.25 19.25) (end 89 43.75) (stroke (width 0.05) (type default)) (fill none) (layer "Edge.Cuts"))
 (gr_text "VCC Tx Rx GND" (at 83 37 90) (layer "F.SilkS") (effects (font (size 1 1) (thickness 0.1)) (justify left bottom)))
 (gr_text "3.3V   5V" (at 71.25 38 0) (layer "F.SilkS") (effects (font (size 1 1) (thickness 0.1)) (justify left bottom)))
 (segment (start 67.2 32.25) (end 65.52 32.25) (width 0.2) (layer "F.Cu") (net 1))
 (segment (start 64.006208 27.647629) (end 64.264548 27.389289) (width 0.4) (layer "F.Cu") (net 1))
 (segment (start 59.25 24.75) (end 59.05 24.95) (width 0.4) (layer "F.Cu") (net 1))
 (segment (start 65.8 32.53) (end 65.18 31.91) (width 0.4) (layer "F.Cu") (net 1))
 (segment (start 56 35) (end 55.275 34.275) (width 0.4) (layer "F.Cu") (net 1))
 (segment (start 62.5 41.5625) (end 56.75 35.8125) (width 0.4) (layer "F.Cu") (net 1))
 (segment (start 65.52 32.25) (end 65.18 31.91) (width 0.2) (layer "F.Cu") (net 1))
 (segment (start 64.05 31.91) (end 65.18 31.91) (width 0.2) (layer "F.Cu") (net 1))
 (segment (start 56.7 25.25) (end 57 24.95) (width 0.2) (layer "F.Cu") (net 1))
 (segment (start 52.93 24.75) (end 52.93 25.25) (width 0.2) (layer "F.Cu") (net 1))
 (segment (start 64.335259 27.46) (end 62.5 29.295259) (width 0.2) (layer "F.Cu") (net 1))
 (segment (start 50.93 34.75) (end 49.23 33.05) (width 0.2) (layer "F.Cu") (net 1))
 (segment (start 57 32.55) (end 55.275 34.275) (width 0.2) (layer "F.Cu") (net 1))
 (segment (start 50.93 22.75) (end 52.93 24.75) (width 0.2) (layer "F.Cu") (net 1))
 (segment (start 52.93 25.25) (end 56.7 25.25) (width 0.2) (layer "F.Cu") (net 1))
 (segment (start 59.25 24.75) (end 62.147629 27.647629) (width 0.4) (layer "F.Cu") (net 1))
 (segment (start 49.23 24.45) (end 50.93 22.75) (width 0.2) (layer "F.Cu") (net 1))
 (segment (start 56.75 35) (end 56 35) (width 0.4) (layer "F.Cu") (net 1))
 (segment (start 56.75 35.8125) (end 56.75 35) (width 0.4) (layer "F.Cu") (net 1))
 (segment (start 65.8 33.75) (end 65.8 32.53) (width 0.4) (layer "F.Cu") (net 1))
 (segment (start 49.23 33.05) (end 49.23 24.45) (width 0.2) (layer "F.Cu") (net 1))
 (segment (start 85 27.46) (end 64.335259 27.46) (width 0.2) (layer "F.Cu") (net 1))
 (segment (start 62.5 21.5) (end 59.25 24.75) (width 0.4) (layer "F.Cu") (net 1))
 (segment (start 62.147629 27.647629) (end 64.006208 27.647629) (width 0.4) (layer "F.Cu") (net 1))
 (segment (start 59.05 24.95) (end 57 24.95) (width 0.4) (layer "F.Cu") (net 1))
 (segment (start 62.5 30.36) (end 64.05 31.91) (width 0.2) (layer "F.Cu") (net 1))
 (segment (start 62.5 29.295259) (end 62.5 30.36) (width 0.2) (layer "F.Cu") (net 1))
 (segment (start 54.8 34.75) (end 50.93 34.75) (width 0.2) (layer "F.Cu") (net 1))
 (segment (start 55.275 34.275) (end 54.8 34.75) (width 0.2) (layer "F.Cu") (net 1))
 (segment (start 58.497629 31.747629) (end 59.615258 30.63) (width 0.2) (layer "F.Cu") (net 7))
 (segment (start 59.205 30.63) (end 58.59 31.245) (width 0.2) (layer "F.Cu") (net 7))
 (segment (start 77.62 35) (end 76.47 36.15) (width 0.2) (layer "F.Cu") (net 7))
 (segment (start 58.445259 31.8) (end 58.497629 31.747629) (width 0.2) (layer "F.Cu") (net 7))
 (segment (start 59.82 30.63) (end 59.205 30.63) (width 0.2) (layer "F.Cu") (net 7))
 (segment (start 62.575259 36.15) (end 58.59 32.164741) (width 0.2) (layer "F.Cu") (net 7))
 (segment (start 64.25 33.75) (end 61.13 30.63) (width 0.4) (layer "F.Cu") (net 7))
 (segment (start 61.13 30.63) (end 59.82 30.63) (width 0.4) (layer "F.Cu") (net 7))
 (segment (start 75.1825 37.4375) (end 77.62 35) (width 0.2) (layer "F.Cu") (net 7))
 (segment (start 76.47 36.15) (end 62.575259 36.15) (width 0.2) (layer "F.Cu") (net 7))
 (segment (start 62.5 37.4375) (end 75.1825 37.4375) (width 0.2) (layer "F.Cu") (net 7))
 (segment (start 58.3 33.8175) (end 58.3 35) (width 0.2) (layer "F.Cu") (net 7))
 (segment (start 58.59 33.5275) (end 62.5 37.4375) (width 0.2) (layer "F.Cu") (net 7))
 (segment (start 59.615258 30.63) (end 59.82 30.63) (width 0.2) (layer "F.Cu") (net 7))
 (segment (start 58.59 32.164741) (end 58.59 31.245) (width 0.2) (layer "F.Cu") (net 7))
 (segment (start 58.59 31.245) (end 58.59 33.5275) (width 0.2) (layer "F.Cu") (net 7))
 (segment (start 58.59 33.5275) (end 58.3 33.8175) (width 0.2) (layer "F.Cu") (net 7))
 (segment (start 52.93 32.25) (end 53.38 31.8) (width 0.2) (layer "F.Cu") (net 7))
 (segment (start 53.38 31.8) (end 58.445259 31.8) (width 0.2) (layer "F.Cu") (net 7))
 (segment (start 64.565 29.37) (end 63.95 29.985) (width 0.2) (layer "F.Cu") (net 3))
 (segment (start 65.18 29.37) (end 64.565 29.37) (width 0.2) (layer "F.Cu") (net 3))
 (segment (start 63.95 29.985) (end 63.95 30.884741) (width 0.2) (layer "F.Cu") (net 3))
 (segment (start 68.75 32.25) (end 68.75 31.245) (width 0.2) (layer "F.Cu") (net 3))
 (segment (start 75 31.245) (end 81.165 31.245) (width 0.2) (layer "F.Cu") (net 3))
 (segment (start 75.08 35) (end 75.08 31.325) (width 0.2) (layer "F.Cu") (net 3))
 (segment (start 75.08 31.325) (end 75 31.245) (width 0.2) (layer "F.Cu") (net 3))
 (segment (start 68.75 31.245) (end 75 31.245) (width 0.2) (layer "F.Cu") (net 3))
 (segment (start 81.165 31.245) (end 85 35.08) (width 0.2) (layer "F.Cu") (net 3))
 (segment (start 63.95 30.884741) (end 64.310259 31.245) (width 0.2) (layer "F.Cu") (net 3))
 (segment (start 64.310259 31.245) (end 68.75 31.245) (width 0.2) (layer "F.Cu") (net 3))
 (segment (start 63 26.75) (end 63 26.5) (width 0.4) (layer "F.Cu") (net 8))
 (segment (start 62.5 26) (end 63 26.75) (width 0.4) (layer "F.Cu") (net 8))
 (segment (start 61.33 33.42) (end 59.82 31.91) (width 0.2) (layer "F.Cu") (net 8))
 (segment (start 62.5 25.1) (end 62.5 26) (width 0.4) (layer "F.Cu") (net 8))
 (segment (start 62.91 35) (end 61.33 33.42) (width 0.2) (layer "F.Cu") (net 8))
 (segment (start 72.54 35) (end 62.91 35) (width 0.2) (layer "F.Cu") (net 8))
 (via (at 63 26.75) (size 0.6) (drill 0.3) (layers "F.Cu" "B.Cu") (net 8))
 (via (at 61.33 33.42) (size 0.6) (drill 0.3) (layers "F.Cu" "B.Cu") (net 8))
 (segment (start 63 31.75) (end 61.33 33.42) (width 0.4) (layer "B.Cu") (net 8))
 (segment (start 63 26.75) (end 63 31.75) (width 0.4) (layer "B.Cu") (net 8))
 (segment (start 59.72 28) (end 59.82 28.1) (width 0.2) (layer "F.Cu") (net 5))
 (segment (start 57.15 28) (end 57.15 26.65) (width 0.2) (layer "F.Cu") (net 5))
 (segment (start 57.15 28) (end 59.72 28) (width 0.2) (layer "F.Cu") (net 5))
 (segment (start 57.15 26.65) (end 57 26.5) (width 0.2) (layer "F.Cu") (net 5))
 (segment (start 57 29.65) (end 57.15 29.5) (width 0.2) (layer "F.Cu") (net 6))
 (segment (start 57 31) (end 57 29.65) (width 0.2) (layer "F.Cu") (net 6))
 (segment (start 59.69 29.5) (end 59.82 29.37) (width 0.2) (layer "F.Cu") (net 6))
 (segment (start 57.15 29.5) (end 59.69 29.5) (width 0.2) (layer "F.Cu") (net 6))
 (segment (start 65.18 28.1) (end 83.1 28.1) (width 0.2) (layer "F.Cu") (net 4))
 (segment (start 83.1 28.1) (end 85 30) (width 0.2) (layer "F.Cu") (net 4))
 (segment (start 65.18 30.63) (end 83.09 30.63) (width 0.2) (layer "F.Cu") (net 2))
 (segment (start 83.09 30.63) (end 85 32.54) (width 0.2) (layer "F.Cu") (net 2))
 (segment (start 52.93 27.75) (end 55.25 27.75) (width 0.2) (layer "F.Cu") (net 13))
 (segment (start 55.25 27.75) (end 55.5 28) (width 0.2) (layer "F.Cu") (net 13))
 (segment (start 52.93 29.75) (end 55.25 29.75) (width 0.2) (layer "F.Cu") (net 14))
 (segment (start 55.25 29.75) (end 55.5 29.5) (width 0.2) (layer "F.Cu") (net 14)))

